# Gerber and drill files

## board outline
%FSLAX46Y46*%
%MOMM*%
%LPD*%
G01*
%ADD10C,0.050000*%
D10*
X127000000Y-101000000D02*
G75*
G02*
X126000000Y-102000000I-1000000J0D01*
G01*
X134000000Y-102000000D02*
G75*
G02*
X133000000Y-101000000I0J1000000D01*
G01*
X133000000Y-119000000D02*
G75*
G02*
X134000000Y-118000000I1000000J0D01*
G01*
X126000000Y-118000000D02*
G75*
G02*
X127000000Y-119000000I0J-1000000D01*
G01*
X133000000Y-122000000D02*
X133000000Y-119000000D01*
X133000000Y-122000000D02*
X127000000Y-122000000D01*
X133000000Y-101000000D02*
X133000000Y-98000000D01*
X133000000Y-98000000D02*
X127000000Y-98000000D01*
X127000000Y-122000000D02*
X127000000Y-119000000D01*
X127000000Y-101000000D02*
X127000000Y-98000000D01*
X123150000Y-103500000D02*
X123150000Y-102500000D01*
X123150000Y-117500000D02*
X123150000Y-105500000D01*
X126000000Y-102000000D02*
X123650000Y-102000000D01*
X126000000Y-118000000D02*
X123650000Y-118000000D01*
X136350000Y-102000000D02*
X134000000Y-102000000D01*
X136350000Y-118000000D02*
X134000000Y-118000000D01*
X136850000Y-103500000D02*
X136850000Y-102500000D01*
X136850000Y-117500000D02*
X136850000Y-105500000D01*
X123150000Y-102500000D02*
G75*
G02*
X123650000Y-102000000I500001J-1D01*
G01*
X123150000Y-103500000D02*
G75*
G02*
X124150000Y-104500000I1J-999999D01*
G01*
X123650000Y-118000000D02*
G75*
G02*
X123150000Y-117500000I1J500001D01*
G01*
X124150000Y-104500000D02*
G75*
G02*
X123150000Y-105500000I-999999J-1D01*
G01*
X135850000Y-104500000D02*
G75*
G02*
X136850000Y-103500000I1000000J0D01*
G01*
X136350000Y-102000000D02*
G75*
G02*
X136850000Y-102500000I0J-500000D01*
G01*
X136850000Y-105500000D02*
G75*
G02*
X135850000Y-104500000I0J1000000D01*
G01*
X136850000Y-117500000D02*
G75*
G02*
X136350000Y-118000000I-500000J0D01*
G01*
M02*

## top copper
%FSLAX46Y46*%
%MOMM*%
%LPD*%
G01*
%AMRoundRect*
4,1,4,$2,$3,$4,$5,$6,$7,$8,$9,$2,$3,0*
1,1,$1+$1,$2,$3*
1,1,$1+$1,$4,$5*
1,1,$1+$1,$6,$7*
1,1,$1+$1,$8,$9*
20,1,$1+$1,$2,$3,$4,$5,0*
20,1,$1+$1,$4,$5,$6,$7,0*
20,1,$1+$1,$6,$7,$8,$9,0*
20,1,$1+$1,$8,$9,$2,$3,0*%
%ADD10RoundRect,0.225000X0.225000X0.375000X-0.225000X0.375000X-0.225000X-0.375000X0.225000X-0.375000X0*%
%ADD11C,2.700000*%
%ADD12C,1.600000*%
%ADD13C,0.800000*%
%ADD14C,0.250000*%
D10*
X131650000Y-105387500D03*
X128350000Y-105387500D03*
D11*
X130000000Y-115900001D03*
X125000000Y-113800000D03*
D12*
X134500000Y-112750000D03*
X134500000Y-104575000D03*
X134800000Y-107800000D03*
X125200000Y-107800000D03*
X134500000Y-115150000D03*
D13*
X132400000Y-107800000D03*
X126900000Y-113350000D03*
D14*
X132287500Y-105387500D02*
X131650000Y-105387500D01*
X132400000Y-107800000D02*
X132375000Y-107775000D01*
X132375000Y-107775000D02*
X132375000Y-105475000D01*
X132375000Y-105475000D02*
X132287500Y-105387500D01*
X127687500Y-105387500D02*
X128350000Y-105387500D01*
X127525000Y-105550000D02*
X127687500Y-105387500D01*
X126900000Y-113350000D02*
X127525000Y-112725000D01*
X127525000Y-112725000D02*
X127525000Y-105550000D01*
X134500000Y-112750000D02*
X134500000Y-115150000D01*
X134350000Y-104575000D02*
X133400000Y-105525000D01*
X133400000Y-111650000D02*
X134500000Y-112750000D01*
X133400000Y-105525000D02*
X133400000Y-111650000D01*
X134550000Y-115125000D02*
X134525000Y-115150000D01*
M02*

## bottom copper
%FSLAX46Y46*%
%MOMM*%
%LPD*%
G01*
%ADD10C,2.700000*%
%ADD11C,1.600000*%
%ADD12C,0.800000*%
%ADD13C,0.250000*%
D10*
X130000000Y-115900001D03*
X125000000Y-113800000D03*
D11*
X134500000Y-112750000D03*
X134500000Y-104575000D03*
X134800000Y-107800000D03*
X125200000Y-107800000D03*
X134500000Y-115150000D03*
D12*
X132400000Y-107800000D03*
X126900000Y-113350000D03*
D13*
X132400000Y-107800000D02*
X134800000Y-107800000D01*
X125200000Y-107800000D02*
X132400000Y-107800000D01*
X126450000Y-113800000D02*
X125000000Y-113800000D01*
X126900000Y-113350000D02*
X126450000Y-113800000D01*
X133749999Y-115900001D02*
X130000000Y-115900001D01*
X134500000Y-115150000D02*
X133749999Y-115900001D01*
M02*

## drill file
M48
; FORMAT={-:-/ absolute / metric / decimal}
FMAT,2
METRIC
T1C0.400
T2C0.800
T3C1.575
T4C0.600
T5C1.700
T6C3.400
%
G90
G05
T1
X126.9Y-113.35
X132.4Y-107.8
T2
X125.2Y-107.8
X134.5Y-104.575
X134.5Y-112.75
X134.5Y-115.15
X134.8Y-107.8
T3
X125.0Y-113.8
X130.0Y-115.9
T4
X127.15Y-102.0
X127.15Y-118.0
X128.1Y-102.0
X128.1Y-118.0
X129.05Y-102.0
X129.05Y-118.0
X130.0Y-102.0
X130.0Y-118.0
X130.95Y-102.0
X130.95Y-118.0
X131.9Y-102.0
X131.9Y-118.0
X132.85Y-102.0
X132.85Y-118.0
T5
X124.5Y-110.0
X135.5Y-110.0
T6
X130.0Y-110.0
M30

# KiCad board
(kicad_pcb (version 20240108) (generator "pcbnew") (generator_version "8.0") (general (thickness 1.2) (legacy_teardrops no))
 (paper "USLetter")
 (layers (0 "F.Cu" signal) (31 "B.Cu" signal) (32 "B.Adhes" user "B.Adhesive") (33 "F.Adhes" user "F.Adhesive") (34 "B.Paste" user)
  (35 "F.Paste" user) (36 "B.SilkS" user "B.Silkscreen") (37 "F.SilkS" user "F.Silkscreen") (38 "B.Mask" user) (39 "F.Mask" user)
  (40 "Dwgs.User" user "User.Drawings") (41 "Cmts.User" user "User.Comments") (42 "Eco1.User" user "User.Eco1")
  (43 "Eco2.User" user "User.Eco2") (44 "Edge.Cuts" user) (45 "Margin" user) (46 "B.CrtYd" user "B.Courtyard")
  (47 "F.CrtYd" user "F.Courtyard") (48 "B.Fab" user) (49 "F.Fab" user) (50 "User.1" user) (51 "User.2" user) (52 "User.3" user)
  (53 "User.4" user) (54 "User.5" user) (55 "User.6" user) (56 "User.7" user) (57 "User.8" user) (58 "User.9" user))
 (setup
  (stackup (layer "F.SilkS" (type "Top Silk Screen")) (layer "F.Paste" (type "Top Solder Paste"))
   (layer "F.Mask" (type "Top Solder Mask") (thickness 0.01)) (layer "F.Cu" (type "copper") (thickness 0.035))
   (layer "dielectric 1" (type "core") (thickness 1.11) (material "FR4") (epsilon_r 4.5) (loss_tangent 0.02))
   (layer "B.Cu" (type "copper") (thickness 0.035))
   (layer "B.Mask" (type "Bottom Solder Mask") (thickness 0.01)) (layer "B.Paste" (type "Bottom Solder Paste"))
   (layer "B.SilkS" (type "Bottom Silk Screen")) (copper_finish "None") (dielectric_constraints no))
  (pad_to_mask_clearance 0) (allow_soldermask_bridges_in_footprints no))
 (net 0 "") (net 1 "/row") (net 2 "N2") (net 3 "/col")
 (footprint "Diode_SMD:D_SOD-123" (layer "F.Cu") (at 130 105.3875 180)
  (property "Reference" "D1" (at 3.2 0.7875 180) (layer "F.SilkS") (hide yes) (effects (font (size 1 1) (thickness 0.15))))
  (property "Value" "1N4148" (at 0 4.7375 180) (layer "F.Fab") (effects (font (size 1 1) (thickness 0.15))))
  (pad "1" smd roundrect (at -1.65 0 180) (size 0.9 1.2) (layers "F.Cu" "F.Paste" "F.Mask") (roundrect_rratio 0.25) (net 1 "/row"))
  (pad "2" smd roundrect (at 1.65 0 180) (size 0.9 1.2) (layers "F.Cu" "F.Paste" "F.Mask") (roundrect_rratio 0.25) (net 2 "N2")))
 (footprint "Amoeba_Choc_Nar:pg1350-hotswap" (layer "F.Cu") (at 130 110)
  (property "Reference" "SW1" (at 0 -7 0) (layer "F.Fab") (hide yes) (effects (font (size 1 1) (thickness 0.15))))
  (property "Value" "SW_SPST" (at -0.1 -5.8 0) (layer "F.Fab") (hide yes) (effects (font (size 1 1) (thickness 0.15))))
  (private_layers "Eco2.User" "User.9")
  (fp_line (start -6.85 -6.5) (end -6.85 -7.5) (stroke (width 0.05) (type solid)) (layer "Edge.Cuts"))
  (fp_line (start -6.85 7.5) (end -6.85 -4.5) (stroke (width 0.05) (type solid)) (layer "Edge.Cuts"))
  (fp_line (start -4 -8) (end -6.35 -8) (stroke (width 0.05) (type solid)) (layer "Edge.Cuts"))
  (fp_line (start -4 8) (end -6.35 8) (stroke (width 0.05) (type solid)) (layer "Edge.Cuts"))
  (fp_line (start 6.35 -8) (end 4 -8) (stroke (width 0.05) (type solid)) (layer "Edge.Cuts"))
  (fp_line (start 6.35 8) (end 4 8) (stroke (width 0.05) (type solid)) (layer "Edge.Cuts"))
  (fp_line (start 6.85 -6.5) (end 6.85 -7.5) (stroke (width 0.05) (type solid)) (layer "Edge.Cuts"))
  (fp_line (start 6.85 7.5) (end 6.85 -4.5) (stroke (width 0.05) (type solid)) (layer "Edge.Cuts"))
  (fp_arc (start -6.85 -7.5) (mid -6.703553 -7.853553) (end -6.35 -8) (stroke (width 0.05) (type default)) (layer "Edge.Cuts"))
  (fp_arc (start -6.85 -6.5) (mid -6.142893 -6.207107) (end -5.85 -5.5) (stroke (width 0.05) (type default)) (layer "Edge.Cuts"))
  (fp_arc (start -6.35 8) (mid -6.703553 7.853553) (end -6.85 7.5) (stroke (width 0.05) (type default)) (layer "Edge.Cuts"))
  (fp_arc (start -5.85 -5.5) (mid -6.142893 -4.792893) (end -6.85 -4.5) (stroke (width 0.05) (type default)) (layer "Edge.Cuts"))
  (fp_arc (start 5.85 -5.5) (mid 6.142893 -6.207107) (end 6.85 -6.5) (stroke (width 0.05) (type default)) (layer "Edge.Cuts"))
  (fp_arc (start 6.35 -8) (mid 6.703553 -7.853553) (end 6.85 -7.5) (stroke (width 0.05) (type default)) (layer "Edge.Cuts"))
  (fp_arc (start 6.85 -4.5) (mid 6.142893 -4.792893) (end 5.85 -5.5) (stroke (width 0.05) (type default)) (layer "Edge.Cuts"))
  (fp_arc (start 6.85 7.5) (mid 6.703553 7.853553) (end 6.35 8) (stroke (width 0.05) (type default)) (layer "Edge.Cuts"))
  (pad "" np_thru_hole circle (at -5.5 0 180) (size 1.7 1.7) (drill 1.7) (layers "*.Cu" "*.Mask"))
  (pad "" np_thru_hole circle (at 0 0 180) (size 3.4 3.4) (drill 3.4) (layers "*.Cu" "*.Mask"))
  (pad "" np_thru_hole circle (at 5.5 0 180) (size 1.7 1.7) (drill 1.7) (layers "*.Cu" "*.Mask"))
  (pad "1" thru_hole circle (at 0 5.900001 180) (size 2.7 2.7) (drill 1.5748) (layers "*.Cu" "*.Mask") (remove_unused_layers no)
   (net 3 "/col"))
  (pad "2" thru_hole circle (at -5 3.8 180) (size 2.7 2.7) (drill 1.5748) (layers "*.Cu" "*.Mask") (remove_unused_layers no) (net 2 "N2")))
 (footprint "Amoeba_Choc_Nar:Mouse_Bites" (layer "F.Cu") (at 130 118)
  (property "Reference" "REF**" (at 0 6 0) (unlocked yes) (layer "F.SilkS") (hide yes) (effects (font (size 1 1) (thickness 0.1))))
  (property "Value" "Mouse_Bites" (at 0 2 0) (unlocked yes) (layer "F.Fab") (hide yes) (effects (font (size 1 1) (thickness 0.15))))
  (pad "" np_thru_hole circle (at -2.85 0) (size 0.6 0.6) (drill 0.6) (layers "*.Mask"))
  (pad "" np_thru_hole circle (at -1.9 0) (size 0.6 0.6) (drill 0.6) (layers "*.Mask"))
  (pad "" np_thru_hole circle (at -0.95 0) (size 0.6 0.6) (drill 0.6) (layers "*.Mask"))
  (pad "" np_thru_hole circle (at 0 0) (size 0.6 0.6) (drill 0.6) (layers "*.Mask"))
  (pad "" np_thru_hole circle (at 0.95 0) (size 0.6 0.6) (drill 0.6) (layers "*.Mask"))
  (pad "" np_thru_hole circle (at 1.9 0) (size 0.6 0.6) (drill 0.6) (layers "*.Mask"))
  (pad "" np_thru_hole circle (at 2.85 0) (size 0.6 0.6) (drill 0.6) (layers "*.Mask")))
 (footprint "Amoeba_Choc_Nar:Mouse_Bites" (layer "F.Cu") (at 130 102)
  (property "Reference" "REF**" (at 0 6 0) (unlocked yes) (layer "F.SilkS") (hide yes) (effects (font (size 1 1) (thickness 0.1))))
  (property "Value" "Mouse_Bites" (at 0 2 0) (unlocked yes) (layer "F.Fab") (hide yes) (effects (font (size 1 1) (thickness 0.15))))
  (pad "" np_thru_hole circle (at -2.85 0) (size 0.6 0.6) (drill 0.6) (layers "*.Mask"))
  (pad "" np_thru_hole circle (at -1.9 0) (size 0.6 0.6) (drill 0.6) (layers "*.Mask"))
  (pad "" np_thru_hole circle (at -0.95 0) (size 0.6 0.6) (drill 0.6) (layers "*.Mask"))
  (pad "" np_thru_hole circle (at 0 0) (size 0.6 0.6) (drill 0.6) (layers "*.Mask"))
  (pad "" np_thru_hole circle (at 0.95 0) (size 0.6 0.6) (drill 0.6) (layers "*.Mask"))
  (pad "" np_thru_hole circle (at 1.9 0) (size 0.6 0.6) (drill 0.6) (layers "*.Mask"))
  (pad "" np_thru_hole circle (at 2.85 0) (size 0.6 0.6) (drill 0.6) (layers "*.Mask")))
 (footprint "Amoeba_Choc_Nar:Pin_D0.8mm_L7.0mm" (layer "B.Cu") (at 134.5 112.75 180)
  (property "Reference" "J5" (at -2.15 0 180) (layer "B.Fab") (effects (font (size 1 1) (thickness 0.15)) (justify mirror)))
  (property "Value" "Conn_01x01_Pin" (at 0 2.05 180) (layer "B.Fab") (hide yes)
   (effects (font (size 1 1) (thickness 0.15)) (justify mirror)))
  (pad "1" thru_hole circle (at 0 0 180) (size 1.6 1.6) (drill 0.8) (layers "*.Cu" "*.Mask") (remove_unused_layers no) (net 3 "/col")))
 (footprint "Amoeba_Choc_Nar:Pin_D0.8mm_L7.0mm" (layer "B.Cu") (at 134.5 104.575 180)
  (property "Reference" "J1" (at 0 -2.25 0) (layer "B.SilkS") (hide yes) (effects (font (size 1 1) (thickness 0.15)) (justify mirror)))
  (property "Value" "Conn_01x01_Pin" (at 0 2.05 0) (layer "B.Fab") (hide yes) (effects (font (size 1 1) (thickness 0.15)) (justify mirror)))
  (pad "1" thru_hole circle (at 0 0 180) (size 1.6 1.6) (drill 0.8) (layers "*.Cu" "*.Mask") (remove_unused_layers no) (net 3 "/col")))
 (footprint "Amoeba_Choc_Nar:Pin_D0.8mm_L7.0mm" (layer "B.Cu") (at 134.8 107.8 180)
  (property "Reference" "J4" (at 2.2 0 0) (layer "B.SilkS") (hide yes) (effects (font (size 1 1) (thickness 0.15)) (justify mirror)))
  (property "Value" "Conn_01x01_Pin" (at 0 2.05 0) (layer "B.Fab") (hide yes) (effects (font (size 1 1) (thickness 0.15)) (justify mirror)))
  (pad "1" thru_hole circle (at 0 0 180) (size 1.6 1.6) (drill 0.8) (layers "*.Cu" "*.Mask") (remove_unused_layers no) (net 1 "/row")))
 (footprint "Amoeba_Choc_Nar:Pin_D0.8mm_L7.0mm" (layer "B.Cu") (at 125.2 107.8 180)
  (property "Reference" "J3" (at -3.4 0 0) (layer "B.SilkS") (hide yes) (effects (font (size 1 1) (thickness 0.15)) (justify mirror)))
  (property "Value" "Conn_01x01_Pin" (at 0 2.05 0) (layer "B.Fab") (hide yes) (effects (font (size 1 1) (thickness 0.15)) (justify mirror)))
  (pad "1" thru_hole circle (at 0 0 180) (size 1.6 1.6) (drill 0.8) (layers "*.Cu" "*.Mask") (remove_unused_layers no) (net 1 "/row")))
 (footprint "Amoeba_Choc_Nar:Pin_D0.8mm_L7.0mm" (layer "B.Cu") (at 134.5 115.15 180)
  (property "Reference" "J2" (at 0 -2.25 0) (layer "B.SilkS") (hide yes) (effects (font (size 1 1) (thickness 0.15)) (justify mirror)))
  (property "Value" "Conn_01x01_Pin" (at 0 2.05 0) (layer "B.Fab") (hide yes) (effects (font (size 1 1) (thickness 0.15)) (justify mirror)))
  (pad "1" thru_hole circle (at 0 0 180) (size 1.6 1.6) (drill 0.8) (layers "*.Cu" "*.Mask") (remove_unused_layers no) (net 3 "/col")))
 (gr_arc (start 127 101) (mid 126.707107 101.707107) (end 126 102) (stroke (width 0.05) (type default)) (layer "Edge.Cuts"))
 (gr_arc (start 134 102) (mid 133.292893 101.707107) (end 133 101) (stroke (width 0.05) (type default)) (layer "Edge.Cuts"))
 (gr_arc (start 133 119) (mid 133.292893 118.292893) (end 134 118) (stroke (width 0.05) (type default)) (layer "Edge.Cuts"))
 (gr_arc (start 126 118) (mid 126.707107 118.292893) (end 127 119) (stroke (width 0.05) (type default)) (layer "Edge.Cuts"))
 (gr_line (start 133 122) (end 133 119) (stroke (width 0.05) (type default)) (layer "Edge.Cuts"))
 (gr_line (start 133 122) (end 127 122) (stroke (width 0.05) (type default)) (layer "Edge.Cuts"))
 (gr_line (start 133 101) (end 133 98) (stroke (width 0.05) (type default)) (layer "Edge.Cuts"))
 (gr_line (start 133 98) (end 127 98) (stroke (width 0.05) (type default)) (layer "Edge.Cuts"))
 (gr_line (start 127 122) (end 127 119) (stroke (width 0.05) (type default)) (layer "Edge.Cuts"))
 (gr_line (start 127 101) (end 127 98) (stroke (width 0.05) (type default)) (layer "Edge.Cuts"))
 (segment (start 132.2875 105.3875) (end 131.65 105.3875) (width 0.25) (layer "F.Cu") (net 1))
 (segment (start 132.4 107.8) (end 132.375 107.775) (width 0.25) (layer "F.Cu") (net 1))
 (segment (start 132.375 107.775) (end 132.375 105.475) (width 0.25) (layer "F.Cu") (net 1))
 (segment (start 132.375 105.475) (end 132.2875 105.3875) (width 0.25) (layer "F.Cu") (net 1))
 (via (at 132.4 107.8) (size 0.8) (drill 0.4) (layers "F.Cu" "B.Cu") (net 1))
 (segment (start 132.4 107.8) (end 134.8 107.8) (width 0.25) (layer "B.Cu") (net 1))
 (segment (start 125.2 107.8) (end 132.4 107.8) (width 0.25) (layer "B.Cu") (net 1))
 (segment (start 127.6875 105.3875) (end 128.35 105.3875) (width 0.25) (layer "F.Cu") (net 2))
 (segment (start 127.525 105.55) (end 127.6875 105.3875) (width 0.25) (layer "F.Cu") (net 2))
 (segment (start 126.9 113.35) (end 127.525 112.725) (width 0.25) (layer "F.Cu") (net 2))
 (segment (start 127.525 112.725) (end 127.525 105.55) (width 0.25) (layer "F.Cu") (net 2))
 (via (at 126.9 113.35) (size 0.8) (drill 0.4) (layers "F.Cu" "B.Cu") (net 2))
 (segment (start 126.45 113.8) (end 125 113.8) (width 0.25) (layer "B.Cu") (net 2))
 (segment (start 126.9 113.35) (end 126.45 113.8) (width 0.25) (layer "B.Cu") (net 2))
 (segment (start 134.5 112.75) (end 134.5 115.15) (width 0.25) (layer "F.Cu") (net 3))
 (segment (start 134.35 104.575) (end 133.4 105.525) (width 0.25) (layer "F.Cu") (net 3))
 (segment (start 133.4 111.65) (end 134.5 112.75) (width 0.25) (layer "F.Cu") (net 3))
 (segment (start 133.4 105.525) (end 133.4 111.65) (width 0.25) (layer "F.Cu") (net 3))
 (segment (start 134.55 115.125) (end 134.525 115.15) (width 0.25) (layer "F.Cu") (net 3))
 (segment (start 133.749999 115.900001) (end 130 115.900001) (width 0.25) (layer "B.Cu") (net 3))
 (segment (start 134.5 115.15) (end 133.749999 115.900001) (width 0.25) (layer "B.Cu") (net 3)))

